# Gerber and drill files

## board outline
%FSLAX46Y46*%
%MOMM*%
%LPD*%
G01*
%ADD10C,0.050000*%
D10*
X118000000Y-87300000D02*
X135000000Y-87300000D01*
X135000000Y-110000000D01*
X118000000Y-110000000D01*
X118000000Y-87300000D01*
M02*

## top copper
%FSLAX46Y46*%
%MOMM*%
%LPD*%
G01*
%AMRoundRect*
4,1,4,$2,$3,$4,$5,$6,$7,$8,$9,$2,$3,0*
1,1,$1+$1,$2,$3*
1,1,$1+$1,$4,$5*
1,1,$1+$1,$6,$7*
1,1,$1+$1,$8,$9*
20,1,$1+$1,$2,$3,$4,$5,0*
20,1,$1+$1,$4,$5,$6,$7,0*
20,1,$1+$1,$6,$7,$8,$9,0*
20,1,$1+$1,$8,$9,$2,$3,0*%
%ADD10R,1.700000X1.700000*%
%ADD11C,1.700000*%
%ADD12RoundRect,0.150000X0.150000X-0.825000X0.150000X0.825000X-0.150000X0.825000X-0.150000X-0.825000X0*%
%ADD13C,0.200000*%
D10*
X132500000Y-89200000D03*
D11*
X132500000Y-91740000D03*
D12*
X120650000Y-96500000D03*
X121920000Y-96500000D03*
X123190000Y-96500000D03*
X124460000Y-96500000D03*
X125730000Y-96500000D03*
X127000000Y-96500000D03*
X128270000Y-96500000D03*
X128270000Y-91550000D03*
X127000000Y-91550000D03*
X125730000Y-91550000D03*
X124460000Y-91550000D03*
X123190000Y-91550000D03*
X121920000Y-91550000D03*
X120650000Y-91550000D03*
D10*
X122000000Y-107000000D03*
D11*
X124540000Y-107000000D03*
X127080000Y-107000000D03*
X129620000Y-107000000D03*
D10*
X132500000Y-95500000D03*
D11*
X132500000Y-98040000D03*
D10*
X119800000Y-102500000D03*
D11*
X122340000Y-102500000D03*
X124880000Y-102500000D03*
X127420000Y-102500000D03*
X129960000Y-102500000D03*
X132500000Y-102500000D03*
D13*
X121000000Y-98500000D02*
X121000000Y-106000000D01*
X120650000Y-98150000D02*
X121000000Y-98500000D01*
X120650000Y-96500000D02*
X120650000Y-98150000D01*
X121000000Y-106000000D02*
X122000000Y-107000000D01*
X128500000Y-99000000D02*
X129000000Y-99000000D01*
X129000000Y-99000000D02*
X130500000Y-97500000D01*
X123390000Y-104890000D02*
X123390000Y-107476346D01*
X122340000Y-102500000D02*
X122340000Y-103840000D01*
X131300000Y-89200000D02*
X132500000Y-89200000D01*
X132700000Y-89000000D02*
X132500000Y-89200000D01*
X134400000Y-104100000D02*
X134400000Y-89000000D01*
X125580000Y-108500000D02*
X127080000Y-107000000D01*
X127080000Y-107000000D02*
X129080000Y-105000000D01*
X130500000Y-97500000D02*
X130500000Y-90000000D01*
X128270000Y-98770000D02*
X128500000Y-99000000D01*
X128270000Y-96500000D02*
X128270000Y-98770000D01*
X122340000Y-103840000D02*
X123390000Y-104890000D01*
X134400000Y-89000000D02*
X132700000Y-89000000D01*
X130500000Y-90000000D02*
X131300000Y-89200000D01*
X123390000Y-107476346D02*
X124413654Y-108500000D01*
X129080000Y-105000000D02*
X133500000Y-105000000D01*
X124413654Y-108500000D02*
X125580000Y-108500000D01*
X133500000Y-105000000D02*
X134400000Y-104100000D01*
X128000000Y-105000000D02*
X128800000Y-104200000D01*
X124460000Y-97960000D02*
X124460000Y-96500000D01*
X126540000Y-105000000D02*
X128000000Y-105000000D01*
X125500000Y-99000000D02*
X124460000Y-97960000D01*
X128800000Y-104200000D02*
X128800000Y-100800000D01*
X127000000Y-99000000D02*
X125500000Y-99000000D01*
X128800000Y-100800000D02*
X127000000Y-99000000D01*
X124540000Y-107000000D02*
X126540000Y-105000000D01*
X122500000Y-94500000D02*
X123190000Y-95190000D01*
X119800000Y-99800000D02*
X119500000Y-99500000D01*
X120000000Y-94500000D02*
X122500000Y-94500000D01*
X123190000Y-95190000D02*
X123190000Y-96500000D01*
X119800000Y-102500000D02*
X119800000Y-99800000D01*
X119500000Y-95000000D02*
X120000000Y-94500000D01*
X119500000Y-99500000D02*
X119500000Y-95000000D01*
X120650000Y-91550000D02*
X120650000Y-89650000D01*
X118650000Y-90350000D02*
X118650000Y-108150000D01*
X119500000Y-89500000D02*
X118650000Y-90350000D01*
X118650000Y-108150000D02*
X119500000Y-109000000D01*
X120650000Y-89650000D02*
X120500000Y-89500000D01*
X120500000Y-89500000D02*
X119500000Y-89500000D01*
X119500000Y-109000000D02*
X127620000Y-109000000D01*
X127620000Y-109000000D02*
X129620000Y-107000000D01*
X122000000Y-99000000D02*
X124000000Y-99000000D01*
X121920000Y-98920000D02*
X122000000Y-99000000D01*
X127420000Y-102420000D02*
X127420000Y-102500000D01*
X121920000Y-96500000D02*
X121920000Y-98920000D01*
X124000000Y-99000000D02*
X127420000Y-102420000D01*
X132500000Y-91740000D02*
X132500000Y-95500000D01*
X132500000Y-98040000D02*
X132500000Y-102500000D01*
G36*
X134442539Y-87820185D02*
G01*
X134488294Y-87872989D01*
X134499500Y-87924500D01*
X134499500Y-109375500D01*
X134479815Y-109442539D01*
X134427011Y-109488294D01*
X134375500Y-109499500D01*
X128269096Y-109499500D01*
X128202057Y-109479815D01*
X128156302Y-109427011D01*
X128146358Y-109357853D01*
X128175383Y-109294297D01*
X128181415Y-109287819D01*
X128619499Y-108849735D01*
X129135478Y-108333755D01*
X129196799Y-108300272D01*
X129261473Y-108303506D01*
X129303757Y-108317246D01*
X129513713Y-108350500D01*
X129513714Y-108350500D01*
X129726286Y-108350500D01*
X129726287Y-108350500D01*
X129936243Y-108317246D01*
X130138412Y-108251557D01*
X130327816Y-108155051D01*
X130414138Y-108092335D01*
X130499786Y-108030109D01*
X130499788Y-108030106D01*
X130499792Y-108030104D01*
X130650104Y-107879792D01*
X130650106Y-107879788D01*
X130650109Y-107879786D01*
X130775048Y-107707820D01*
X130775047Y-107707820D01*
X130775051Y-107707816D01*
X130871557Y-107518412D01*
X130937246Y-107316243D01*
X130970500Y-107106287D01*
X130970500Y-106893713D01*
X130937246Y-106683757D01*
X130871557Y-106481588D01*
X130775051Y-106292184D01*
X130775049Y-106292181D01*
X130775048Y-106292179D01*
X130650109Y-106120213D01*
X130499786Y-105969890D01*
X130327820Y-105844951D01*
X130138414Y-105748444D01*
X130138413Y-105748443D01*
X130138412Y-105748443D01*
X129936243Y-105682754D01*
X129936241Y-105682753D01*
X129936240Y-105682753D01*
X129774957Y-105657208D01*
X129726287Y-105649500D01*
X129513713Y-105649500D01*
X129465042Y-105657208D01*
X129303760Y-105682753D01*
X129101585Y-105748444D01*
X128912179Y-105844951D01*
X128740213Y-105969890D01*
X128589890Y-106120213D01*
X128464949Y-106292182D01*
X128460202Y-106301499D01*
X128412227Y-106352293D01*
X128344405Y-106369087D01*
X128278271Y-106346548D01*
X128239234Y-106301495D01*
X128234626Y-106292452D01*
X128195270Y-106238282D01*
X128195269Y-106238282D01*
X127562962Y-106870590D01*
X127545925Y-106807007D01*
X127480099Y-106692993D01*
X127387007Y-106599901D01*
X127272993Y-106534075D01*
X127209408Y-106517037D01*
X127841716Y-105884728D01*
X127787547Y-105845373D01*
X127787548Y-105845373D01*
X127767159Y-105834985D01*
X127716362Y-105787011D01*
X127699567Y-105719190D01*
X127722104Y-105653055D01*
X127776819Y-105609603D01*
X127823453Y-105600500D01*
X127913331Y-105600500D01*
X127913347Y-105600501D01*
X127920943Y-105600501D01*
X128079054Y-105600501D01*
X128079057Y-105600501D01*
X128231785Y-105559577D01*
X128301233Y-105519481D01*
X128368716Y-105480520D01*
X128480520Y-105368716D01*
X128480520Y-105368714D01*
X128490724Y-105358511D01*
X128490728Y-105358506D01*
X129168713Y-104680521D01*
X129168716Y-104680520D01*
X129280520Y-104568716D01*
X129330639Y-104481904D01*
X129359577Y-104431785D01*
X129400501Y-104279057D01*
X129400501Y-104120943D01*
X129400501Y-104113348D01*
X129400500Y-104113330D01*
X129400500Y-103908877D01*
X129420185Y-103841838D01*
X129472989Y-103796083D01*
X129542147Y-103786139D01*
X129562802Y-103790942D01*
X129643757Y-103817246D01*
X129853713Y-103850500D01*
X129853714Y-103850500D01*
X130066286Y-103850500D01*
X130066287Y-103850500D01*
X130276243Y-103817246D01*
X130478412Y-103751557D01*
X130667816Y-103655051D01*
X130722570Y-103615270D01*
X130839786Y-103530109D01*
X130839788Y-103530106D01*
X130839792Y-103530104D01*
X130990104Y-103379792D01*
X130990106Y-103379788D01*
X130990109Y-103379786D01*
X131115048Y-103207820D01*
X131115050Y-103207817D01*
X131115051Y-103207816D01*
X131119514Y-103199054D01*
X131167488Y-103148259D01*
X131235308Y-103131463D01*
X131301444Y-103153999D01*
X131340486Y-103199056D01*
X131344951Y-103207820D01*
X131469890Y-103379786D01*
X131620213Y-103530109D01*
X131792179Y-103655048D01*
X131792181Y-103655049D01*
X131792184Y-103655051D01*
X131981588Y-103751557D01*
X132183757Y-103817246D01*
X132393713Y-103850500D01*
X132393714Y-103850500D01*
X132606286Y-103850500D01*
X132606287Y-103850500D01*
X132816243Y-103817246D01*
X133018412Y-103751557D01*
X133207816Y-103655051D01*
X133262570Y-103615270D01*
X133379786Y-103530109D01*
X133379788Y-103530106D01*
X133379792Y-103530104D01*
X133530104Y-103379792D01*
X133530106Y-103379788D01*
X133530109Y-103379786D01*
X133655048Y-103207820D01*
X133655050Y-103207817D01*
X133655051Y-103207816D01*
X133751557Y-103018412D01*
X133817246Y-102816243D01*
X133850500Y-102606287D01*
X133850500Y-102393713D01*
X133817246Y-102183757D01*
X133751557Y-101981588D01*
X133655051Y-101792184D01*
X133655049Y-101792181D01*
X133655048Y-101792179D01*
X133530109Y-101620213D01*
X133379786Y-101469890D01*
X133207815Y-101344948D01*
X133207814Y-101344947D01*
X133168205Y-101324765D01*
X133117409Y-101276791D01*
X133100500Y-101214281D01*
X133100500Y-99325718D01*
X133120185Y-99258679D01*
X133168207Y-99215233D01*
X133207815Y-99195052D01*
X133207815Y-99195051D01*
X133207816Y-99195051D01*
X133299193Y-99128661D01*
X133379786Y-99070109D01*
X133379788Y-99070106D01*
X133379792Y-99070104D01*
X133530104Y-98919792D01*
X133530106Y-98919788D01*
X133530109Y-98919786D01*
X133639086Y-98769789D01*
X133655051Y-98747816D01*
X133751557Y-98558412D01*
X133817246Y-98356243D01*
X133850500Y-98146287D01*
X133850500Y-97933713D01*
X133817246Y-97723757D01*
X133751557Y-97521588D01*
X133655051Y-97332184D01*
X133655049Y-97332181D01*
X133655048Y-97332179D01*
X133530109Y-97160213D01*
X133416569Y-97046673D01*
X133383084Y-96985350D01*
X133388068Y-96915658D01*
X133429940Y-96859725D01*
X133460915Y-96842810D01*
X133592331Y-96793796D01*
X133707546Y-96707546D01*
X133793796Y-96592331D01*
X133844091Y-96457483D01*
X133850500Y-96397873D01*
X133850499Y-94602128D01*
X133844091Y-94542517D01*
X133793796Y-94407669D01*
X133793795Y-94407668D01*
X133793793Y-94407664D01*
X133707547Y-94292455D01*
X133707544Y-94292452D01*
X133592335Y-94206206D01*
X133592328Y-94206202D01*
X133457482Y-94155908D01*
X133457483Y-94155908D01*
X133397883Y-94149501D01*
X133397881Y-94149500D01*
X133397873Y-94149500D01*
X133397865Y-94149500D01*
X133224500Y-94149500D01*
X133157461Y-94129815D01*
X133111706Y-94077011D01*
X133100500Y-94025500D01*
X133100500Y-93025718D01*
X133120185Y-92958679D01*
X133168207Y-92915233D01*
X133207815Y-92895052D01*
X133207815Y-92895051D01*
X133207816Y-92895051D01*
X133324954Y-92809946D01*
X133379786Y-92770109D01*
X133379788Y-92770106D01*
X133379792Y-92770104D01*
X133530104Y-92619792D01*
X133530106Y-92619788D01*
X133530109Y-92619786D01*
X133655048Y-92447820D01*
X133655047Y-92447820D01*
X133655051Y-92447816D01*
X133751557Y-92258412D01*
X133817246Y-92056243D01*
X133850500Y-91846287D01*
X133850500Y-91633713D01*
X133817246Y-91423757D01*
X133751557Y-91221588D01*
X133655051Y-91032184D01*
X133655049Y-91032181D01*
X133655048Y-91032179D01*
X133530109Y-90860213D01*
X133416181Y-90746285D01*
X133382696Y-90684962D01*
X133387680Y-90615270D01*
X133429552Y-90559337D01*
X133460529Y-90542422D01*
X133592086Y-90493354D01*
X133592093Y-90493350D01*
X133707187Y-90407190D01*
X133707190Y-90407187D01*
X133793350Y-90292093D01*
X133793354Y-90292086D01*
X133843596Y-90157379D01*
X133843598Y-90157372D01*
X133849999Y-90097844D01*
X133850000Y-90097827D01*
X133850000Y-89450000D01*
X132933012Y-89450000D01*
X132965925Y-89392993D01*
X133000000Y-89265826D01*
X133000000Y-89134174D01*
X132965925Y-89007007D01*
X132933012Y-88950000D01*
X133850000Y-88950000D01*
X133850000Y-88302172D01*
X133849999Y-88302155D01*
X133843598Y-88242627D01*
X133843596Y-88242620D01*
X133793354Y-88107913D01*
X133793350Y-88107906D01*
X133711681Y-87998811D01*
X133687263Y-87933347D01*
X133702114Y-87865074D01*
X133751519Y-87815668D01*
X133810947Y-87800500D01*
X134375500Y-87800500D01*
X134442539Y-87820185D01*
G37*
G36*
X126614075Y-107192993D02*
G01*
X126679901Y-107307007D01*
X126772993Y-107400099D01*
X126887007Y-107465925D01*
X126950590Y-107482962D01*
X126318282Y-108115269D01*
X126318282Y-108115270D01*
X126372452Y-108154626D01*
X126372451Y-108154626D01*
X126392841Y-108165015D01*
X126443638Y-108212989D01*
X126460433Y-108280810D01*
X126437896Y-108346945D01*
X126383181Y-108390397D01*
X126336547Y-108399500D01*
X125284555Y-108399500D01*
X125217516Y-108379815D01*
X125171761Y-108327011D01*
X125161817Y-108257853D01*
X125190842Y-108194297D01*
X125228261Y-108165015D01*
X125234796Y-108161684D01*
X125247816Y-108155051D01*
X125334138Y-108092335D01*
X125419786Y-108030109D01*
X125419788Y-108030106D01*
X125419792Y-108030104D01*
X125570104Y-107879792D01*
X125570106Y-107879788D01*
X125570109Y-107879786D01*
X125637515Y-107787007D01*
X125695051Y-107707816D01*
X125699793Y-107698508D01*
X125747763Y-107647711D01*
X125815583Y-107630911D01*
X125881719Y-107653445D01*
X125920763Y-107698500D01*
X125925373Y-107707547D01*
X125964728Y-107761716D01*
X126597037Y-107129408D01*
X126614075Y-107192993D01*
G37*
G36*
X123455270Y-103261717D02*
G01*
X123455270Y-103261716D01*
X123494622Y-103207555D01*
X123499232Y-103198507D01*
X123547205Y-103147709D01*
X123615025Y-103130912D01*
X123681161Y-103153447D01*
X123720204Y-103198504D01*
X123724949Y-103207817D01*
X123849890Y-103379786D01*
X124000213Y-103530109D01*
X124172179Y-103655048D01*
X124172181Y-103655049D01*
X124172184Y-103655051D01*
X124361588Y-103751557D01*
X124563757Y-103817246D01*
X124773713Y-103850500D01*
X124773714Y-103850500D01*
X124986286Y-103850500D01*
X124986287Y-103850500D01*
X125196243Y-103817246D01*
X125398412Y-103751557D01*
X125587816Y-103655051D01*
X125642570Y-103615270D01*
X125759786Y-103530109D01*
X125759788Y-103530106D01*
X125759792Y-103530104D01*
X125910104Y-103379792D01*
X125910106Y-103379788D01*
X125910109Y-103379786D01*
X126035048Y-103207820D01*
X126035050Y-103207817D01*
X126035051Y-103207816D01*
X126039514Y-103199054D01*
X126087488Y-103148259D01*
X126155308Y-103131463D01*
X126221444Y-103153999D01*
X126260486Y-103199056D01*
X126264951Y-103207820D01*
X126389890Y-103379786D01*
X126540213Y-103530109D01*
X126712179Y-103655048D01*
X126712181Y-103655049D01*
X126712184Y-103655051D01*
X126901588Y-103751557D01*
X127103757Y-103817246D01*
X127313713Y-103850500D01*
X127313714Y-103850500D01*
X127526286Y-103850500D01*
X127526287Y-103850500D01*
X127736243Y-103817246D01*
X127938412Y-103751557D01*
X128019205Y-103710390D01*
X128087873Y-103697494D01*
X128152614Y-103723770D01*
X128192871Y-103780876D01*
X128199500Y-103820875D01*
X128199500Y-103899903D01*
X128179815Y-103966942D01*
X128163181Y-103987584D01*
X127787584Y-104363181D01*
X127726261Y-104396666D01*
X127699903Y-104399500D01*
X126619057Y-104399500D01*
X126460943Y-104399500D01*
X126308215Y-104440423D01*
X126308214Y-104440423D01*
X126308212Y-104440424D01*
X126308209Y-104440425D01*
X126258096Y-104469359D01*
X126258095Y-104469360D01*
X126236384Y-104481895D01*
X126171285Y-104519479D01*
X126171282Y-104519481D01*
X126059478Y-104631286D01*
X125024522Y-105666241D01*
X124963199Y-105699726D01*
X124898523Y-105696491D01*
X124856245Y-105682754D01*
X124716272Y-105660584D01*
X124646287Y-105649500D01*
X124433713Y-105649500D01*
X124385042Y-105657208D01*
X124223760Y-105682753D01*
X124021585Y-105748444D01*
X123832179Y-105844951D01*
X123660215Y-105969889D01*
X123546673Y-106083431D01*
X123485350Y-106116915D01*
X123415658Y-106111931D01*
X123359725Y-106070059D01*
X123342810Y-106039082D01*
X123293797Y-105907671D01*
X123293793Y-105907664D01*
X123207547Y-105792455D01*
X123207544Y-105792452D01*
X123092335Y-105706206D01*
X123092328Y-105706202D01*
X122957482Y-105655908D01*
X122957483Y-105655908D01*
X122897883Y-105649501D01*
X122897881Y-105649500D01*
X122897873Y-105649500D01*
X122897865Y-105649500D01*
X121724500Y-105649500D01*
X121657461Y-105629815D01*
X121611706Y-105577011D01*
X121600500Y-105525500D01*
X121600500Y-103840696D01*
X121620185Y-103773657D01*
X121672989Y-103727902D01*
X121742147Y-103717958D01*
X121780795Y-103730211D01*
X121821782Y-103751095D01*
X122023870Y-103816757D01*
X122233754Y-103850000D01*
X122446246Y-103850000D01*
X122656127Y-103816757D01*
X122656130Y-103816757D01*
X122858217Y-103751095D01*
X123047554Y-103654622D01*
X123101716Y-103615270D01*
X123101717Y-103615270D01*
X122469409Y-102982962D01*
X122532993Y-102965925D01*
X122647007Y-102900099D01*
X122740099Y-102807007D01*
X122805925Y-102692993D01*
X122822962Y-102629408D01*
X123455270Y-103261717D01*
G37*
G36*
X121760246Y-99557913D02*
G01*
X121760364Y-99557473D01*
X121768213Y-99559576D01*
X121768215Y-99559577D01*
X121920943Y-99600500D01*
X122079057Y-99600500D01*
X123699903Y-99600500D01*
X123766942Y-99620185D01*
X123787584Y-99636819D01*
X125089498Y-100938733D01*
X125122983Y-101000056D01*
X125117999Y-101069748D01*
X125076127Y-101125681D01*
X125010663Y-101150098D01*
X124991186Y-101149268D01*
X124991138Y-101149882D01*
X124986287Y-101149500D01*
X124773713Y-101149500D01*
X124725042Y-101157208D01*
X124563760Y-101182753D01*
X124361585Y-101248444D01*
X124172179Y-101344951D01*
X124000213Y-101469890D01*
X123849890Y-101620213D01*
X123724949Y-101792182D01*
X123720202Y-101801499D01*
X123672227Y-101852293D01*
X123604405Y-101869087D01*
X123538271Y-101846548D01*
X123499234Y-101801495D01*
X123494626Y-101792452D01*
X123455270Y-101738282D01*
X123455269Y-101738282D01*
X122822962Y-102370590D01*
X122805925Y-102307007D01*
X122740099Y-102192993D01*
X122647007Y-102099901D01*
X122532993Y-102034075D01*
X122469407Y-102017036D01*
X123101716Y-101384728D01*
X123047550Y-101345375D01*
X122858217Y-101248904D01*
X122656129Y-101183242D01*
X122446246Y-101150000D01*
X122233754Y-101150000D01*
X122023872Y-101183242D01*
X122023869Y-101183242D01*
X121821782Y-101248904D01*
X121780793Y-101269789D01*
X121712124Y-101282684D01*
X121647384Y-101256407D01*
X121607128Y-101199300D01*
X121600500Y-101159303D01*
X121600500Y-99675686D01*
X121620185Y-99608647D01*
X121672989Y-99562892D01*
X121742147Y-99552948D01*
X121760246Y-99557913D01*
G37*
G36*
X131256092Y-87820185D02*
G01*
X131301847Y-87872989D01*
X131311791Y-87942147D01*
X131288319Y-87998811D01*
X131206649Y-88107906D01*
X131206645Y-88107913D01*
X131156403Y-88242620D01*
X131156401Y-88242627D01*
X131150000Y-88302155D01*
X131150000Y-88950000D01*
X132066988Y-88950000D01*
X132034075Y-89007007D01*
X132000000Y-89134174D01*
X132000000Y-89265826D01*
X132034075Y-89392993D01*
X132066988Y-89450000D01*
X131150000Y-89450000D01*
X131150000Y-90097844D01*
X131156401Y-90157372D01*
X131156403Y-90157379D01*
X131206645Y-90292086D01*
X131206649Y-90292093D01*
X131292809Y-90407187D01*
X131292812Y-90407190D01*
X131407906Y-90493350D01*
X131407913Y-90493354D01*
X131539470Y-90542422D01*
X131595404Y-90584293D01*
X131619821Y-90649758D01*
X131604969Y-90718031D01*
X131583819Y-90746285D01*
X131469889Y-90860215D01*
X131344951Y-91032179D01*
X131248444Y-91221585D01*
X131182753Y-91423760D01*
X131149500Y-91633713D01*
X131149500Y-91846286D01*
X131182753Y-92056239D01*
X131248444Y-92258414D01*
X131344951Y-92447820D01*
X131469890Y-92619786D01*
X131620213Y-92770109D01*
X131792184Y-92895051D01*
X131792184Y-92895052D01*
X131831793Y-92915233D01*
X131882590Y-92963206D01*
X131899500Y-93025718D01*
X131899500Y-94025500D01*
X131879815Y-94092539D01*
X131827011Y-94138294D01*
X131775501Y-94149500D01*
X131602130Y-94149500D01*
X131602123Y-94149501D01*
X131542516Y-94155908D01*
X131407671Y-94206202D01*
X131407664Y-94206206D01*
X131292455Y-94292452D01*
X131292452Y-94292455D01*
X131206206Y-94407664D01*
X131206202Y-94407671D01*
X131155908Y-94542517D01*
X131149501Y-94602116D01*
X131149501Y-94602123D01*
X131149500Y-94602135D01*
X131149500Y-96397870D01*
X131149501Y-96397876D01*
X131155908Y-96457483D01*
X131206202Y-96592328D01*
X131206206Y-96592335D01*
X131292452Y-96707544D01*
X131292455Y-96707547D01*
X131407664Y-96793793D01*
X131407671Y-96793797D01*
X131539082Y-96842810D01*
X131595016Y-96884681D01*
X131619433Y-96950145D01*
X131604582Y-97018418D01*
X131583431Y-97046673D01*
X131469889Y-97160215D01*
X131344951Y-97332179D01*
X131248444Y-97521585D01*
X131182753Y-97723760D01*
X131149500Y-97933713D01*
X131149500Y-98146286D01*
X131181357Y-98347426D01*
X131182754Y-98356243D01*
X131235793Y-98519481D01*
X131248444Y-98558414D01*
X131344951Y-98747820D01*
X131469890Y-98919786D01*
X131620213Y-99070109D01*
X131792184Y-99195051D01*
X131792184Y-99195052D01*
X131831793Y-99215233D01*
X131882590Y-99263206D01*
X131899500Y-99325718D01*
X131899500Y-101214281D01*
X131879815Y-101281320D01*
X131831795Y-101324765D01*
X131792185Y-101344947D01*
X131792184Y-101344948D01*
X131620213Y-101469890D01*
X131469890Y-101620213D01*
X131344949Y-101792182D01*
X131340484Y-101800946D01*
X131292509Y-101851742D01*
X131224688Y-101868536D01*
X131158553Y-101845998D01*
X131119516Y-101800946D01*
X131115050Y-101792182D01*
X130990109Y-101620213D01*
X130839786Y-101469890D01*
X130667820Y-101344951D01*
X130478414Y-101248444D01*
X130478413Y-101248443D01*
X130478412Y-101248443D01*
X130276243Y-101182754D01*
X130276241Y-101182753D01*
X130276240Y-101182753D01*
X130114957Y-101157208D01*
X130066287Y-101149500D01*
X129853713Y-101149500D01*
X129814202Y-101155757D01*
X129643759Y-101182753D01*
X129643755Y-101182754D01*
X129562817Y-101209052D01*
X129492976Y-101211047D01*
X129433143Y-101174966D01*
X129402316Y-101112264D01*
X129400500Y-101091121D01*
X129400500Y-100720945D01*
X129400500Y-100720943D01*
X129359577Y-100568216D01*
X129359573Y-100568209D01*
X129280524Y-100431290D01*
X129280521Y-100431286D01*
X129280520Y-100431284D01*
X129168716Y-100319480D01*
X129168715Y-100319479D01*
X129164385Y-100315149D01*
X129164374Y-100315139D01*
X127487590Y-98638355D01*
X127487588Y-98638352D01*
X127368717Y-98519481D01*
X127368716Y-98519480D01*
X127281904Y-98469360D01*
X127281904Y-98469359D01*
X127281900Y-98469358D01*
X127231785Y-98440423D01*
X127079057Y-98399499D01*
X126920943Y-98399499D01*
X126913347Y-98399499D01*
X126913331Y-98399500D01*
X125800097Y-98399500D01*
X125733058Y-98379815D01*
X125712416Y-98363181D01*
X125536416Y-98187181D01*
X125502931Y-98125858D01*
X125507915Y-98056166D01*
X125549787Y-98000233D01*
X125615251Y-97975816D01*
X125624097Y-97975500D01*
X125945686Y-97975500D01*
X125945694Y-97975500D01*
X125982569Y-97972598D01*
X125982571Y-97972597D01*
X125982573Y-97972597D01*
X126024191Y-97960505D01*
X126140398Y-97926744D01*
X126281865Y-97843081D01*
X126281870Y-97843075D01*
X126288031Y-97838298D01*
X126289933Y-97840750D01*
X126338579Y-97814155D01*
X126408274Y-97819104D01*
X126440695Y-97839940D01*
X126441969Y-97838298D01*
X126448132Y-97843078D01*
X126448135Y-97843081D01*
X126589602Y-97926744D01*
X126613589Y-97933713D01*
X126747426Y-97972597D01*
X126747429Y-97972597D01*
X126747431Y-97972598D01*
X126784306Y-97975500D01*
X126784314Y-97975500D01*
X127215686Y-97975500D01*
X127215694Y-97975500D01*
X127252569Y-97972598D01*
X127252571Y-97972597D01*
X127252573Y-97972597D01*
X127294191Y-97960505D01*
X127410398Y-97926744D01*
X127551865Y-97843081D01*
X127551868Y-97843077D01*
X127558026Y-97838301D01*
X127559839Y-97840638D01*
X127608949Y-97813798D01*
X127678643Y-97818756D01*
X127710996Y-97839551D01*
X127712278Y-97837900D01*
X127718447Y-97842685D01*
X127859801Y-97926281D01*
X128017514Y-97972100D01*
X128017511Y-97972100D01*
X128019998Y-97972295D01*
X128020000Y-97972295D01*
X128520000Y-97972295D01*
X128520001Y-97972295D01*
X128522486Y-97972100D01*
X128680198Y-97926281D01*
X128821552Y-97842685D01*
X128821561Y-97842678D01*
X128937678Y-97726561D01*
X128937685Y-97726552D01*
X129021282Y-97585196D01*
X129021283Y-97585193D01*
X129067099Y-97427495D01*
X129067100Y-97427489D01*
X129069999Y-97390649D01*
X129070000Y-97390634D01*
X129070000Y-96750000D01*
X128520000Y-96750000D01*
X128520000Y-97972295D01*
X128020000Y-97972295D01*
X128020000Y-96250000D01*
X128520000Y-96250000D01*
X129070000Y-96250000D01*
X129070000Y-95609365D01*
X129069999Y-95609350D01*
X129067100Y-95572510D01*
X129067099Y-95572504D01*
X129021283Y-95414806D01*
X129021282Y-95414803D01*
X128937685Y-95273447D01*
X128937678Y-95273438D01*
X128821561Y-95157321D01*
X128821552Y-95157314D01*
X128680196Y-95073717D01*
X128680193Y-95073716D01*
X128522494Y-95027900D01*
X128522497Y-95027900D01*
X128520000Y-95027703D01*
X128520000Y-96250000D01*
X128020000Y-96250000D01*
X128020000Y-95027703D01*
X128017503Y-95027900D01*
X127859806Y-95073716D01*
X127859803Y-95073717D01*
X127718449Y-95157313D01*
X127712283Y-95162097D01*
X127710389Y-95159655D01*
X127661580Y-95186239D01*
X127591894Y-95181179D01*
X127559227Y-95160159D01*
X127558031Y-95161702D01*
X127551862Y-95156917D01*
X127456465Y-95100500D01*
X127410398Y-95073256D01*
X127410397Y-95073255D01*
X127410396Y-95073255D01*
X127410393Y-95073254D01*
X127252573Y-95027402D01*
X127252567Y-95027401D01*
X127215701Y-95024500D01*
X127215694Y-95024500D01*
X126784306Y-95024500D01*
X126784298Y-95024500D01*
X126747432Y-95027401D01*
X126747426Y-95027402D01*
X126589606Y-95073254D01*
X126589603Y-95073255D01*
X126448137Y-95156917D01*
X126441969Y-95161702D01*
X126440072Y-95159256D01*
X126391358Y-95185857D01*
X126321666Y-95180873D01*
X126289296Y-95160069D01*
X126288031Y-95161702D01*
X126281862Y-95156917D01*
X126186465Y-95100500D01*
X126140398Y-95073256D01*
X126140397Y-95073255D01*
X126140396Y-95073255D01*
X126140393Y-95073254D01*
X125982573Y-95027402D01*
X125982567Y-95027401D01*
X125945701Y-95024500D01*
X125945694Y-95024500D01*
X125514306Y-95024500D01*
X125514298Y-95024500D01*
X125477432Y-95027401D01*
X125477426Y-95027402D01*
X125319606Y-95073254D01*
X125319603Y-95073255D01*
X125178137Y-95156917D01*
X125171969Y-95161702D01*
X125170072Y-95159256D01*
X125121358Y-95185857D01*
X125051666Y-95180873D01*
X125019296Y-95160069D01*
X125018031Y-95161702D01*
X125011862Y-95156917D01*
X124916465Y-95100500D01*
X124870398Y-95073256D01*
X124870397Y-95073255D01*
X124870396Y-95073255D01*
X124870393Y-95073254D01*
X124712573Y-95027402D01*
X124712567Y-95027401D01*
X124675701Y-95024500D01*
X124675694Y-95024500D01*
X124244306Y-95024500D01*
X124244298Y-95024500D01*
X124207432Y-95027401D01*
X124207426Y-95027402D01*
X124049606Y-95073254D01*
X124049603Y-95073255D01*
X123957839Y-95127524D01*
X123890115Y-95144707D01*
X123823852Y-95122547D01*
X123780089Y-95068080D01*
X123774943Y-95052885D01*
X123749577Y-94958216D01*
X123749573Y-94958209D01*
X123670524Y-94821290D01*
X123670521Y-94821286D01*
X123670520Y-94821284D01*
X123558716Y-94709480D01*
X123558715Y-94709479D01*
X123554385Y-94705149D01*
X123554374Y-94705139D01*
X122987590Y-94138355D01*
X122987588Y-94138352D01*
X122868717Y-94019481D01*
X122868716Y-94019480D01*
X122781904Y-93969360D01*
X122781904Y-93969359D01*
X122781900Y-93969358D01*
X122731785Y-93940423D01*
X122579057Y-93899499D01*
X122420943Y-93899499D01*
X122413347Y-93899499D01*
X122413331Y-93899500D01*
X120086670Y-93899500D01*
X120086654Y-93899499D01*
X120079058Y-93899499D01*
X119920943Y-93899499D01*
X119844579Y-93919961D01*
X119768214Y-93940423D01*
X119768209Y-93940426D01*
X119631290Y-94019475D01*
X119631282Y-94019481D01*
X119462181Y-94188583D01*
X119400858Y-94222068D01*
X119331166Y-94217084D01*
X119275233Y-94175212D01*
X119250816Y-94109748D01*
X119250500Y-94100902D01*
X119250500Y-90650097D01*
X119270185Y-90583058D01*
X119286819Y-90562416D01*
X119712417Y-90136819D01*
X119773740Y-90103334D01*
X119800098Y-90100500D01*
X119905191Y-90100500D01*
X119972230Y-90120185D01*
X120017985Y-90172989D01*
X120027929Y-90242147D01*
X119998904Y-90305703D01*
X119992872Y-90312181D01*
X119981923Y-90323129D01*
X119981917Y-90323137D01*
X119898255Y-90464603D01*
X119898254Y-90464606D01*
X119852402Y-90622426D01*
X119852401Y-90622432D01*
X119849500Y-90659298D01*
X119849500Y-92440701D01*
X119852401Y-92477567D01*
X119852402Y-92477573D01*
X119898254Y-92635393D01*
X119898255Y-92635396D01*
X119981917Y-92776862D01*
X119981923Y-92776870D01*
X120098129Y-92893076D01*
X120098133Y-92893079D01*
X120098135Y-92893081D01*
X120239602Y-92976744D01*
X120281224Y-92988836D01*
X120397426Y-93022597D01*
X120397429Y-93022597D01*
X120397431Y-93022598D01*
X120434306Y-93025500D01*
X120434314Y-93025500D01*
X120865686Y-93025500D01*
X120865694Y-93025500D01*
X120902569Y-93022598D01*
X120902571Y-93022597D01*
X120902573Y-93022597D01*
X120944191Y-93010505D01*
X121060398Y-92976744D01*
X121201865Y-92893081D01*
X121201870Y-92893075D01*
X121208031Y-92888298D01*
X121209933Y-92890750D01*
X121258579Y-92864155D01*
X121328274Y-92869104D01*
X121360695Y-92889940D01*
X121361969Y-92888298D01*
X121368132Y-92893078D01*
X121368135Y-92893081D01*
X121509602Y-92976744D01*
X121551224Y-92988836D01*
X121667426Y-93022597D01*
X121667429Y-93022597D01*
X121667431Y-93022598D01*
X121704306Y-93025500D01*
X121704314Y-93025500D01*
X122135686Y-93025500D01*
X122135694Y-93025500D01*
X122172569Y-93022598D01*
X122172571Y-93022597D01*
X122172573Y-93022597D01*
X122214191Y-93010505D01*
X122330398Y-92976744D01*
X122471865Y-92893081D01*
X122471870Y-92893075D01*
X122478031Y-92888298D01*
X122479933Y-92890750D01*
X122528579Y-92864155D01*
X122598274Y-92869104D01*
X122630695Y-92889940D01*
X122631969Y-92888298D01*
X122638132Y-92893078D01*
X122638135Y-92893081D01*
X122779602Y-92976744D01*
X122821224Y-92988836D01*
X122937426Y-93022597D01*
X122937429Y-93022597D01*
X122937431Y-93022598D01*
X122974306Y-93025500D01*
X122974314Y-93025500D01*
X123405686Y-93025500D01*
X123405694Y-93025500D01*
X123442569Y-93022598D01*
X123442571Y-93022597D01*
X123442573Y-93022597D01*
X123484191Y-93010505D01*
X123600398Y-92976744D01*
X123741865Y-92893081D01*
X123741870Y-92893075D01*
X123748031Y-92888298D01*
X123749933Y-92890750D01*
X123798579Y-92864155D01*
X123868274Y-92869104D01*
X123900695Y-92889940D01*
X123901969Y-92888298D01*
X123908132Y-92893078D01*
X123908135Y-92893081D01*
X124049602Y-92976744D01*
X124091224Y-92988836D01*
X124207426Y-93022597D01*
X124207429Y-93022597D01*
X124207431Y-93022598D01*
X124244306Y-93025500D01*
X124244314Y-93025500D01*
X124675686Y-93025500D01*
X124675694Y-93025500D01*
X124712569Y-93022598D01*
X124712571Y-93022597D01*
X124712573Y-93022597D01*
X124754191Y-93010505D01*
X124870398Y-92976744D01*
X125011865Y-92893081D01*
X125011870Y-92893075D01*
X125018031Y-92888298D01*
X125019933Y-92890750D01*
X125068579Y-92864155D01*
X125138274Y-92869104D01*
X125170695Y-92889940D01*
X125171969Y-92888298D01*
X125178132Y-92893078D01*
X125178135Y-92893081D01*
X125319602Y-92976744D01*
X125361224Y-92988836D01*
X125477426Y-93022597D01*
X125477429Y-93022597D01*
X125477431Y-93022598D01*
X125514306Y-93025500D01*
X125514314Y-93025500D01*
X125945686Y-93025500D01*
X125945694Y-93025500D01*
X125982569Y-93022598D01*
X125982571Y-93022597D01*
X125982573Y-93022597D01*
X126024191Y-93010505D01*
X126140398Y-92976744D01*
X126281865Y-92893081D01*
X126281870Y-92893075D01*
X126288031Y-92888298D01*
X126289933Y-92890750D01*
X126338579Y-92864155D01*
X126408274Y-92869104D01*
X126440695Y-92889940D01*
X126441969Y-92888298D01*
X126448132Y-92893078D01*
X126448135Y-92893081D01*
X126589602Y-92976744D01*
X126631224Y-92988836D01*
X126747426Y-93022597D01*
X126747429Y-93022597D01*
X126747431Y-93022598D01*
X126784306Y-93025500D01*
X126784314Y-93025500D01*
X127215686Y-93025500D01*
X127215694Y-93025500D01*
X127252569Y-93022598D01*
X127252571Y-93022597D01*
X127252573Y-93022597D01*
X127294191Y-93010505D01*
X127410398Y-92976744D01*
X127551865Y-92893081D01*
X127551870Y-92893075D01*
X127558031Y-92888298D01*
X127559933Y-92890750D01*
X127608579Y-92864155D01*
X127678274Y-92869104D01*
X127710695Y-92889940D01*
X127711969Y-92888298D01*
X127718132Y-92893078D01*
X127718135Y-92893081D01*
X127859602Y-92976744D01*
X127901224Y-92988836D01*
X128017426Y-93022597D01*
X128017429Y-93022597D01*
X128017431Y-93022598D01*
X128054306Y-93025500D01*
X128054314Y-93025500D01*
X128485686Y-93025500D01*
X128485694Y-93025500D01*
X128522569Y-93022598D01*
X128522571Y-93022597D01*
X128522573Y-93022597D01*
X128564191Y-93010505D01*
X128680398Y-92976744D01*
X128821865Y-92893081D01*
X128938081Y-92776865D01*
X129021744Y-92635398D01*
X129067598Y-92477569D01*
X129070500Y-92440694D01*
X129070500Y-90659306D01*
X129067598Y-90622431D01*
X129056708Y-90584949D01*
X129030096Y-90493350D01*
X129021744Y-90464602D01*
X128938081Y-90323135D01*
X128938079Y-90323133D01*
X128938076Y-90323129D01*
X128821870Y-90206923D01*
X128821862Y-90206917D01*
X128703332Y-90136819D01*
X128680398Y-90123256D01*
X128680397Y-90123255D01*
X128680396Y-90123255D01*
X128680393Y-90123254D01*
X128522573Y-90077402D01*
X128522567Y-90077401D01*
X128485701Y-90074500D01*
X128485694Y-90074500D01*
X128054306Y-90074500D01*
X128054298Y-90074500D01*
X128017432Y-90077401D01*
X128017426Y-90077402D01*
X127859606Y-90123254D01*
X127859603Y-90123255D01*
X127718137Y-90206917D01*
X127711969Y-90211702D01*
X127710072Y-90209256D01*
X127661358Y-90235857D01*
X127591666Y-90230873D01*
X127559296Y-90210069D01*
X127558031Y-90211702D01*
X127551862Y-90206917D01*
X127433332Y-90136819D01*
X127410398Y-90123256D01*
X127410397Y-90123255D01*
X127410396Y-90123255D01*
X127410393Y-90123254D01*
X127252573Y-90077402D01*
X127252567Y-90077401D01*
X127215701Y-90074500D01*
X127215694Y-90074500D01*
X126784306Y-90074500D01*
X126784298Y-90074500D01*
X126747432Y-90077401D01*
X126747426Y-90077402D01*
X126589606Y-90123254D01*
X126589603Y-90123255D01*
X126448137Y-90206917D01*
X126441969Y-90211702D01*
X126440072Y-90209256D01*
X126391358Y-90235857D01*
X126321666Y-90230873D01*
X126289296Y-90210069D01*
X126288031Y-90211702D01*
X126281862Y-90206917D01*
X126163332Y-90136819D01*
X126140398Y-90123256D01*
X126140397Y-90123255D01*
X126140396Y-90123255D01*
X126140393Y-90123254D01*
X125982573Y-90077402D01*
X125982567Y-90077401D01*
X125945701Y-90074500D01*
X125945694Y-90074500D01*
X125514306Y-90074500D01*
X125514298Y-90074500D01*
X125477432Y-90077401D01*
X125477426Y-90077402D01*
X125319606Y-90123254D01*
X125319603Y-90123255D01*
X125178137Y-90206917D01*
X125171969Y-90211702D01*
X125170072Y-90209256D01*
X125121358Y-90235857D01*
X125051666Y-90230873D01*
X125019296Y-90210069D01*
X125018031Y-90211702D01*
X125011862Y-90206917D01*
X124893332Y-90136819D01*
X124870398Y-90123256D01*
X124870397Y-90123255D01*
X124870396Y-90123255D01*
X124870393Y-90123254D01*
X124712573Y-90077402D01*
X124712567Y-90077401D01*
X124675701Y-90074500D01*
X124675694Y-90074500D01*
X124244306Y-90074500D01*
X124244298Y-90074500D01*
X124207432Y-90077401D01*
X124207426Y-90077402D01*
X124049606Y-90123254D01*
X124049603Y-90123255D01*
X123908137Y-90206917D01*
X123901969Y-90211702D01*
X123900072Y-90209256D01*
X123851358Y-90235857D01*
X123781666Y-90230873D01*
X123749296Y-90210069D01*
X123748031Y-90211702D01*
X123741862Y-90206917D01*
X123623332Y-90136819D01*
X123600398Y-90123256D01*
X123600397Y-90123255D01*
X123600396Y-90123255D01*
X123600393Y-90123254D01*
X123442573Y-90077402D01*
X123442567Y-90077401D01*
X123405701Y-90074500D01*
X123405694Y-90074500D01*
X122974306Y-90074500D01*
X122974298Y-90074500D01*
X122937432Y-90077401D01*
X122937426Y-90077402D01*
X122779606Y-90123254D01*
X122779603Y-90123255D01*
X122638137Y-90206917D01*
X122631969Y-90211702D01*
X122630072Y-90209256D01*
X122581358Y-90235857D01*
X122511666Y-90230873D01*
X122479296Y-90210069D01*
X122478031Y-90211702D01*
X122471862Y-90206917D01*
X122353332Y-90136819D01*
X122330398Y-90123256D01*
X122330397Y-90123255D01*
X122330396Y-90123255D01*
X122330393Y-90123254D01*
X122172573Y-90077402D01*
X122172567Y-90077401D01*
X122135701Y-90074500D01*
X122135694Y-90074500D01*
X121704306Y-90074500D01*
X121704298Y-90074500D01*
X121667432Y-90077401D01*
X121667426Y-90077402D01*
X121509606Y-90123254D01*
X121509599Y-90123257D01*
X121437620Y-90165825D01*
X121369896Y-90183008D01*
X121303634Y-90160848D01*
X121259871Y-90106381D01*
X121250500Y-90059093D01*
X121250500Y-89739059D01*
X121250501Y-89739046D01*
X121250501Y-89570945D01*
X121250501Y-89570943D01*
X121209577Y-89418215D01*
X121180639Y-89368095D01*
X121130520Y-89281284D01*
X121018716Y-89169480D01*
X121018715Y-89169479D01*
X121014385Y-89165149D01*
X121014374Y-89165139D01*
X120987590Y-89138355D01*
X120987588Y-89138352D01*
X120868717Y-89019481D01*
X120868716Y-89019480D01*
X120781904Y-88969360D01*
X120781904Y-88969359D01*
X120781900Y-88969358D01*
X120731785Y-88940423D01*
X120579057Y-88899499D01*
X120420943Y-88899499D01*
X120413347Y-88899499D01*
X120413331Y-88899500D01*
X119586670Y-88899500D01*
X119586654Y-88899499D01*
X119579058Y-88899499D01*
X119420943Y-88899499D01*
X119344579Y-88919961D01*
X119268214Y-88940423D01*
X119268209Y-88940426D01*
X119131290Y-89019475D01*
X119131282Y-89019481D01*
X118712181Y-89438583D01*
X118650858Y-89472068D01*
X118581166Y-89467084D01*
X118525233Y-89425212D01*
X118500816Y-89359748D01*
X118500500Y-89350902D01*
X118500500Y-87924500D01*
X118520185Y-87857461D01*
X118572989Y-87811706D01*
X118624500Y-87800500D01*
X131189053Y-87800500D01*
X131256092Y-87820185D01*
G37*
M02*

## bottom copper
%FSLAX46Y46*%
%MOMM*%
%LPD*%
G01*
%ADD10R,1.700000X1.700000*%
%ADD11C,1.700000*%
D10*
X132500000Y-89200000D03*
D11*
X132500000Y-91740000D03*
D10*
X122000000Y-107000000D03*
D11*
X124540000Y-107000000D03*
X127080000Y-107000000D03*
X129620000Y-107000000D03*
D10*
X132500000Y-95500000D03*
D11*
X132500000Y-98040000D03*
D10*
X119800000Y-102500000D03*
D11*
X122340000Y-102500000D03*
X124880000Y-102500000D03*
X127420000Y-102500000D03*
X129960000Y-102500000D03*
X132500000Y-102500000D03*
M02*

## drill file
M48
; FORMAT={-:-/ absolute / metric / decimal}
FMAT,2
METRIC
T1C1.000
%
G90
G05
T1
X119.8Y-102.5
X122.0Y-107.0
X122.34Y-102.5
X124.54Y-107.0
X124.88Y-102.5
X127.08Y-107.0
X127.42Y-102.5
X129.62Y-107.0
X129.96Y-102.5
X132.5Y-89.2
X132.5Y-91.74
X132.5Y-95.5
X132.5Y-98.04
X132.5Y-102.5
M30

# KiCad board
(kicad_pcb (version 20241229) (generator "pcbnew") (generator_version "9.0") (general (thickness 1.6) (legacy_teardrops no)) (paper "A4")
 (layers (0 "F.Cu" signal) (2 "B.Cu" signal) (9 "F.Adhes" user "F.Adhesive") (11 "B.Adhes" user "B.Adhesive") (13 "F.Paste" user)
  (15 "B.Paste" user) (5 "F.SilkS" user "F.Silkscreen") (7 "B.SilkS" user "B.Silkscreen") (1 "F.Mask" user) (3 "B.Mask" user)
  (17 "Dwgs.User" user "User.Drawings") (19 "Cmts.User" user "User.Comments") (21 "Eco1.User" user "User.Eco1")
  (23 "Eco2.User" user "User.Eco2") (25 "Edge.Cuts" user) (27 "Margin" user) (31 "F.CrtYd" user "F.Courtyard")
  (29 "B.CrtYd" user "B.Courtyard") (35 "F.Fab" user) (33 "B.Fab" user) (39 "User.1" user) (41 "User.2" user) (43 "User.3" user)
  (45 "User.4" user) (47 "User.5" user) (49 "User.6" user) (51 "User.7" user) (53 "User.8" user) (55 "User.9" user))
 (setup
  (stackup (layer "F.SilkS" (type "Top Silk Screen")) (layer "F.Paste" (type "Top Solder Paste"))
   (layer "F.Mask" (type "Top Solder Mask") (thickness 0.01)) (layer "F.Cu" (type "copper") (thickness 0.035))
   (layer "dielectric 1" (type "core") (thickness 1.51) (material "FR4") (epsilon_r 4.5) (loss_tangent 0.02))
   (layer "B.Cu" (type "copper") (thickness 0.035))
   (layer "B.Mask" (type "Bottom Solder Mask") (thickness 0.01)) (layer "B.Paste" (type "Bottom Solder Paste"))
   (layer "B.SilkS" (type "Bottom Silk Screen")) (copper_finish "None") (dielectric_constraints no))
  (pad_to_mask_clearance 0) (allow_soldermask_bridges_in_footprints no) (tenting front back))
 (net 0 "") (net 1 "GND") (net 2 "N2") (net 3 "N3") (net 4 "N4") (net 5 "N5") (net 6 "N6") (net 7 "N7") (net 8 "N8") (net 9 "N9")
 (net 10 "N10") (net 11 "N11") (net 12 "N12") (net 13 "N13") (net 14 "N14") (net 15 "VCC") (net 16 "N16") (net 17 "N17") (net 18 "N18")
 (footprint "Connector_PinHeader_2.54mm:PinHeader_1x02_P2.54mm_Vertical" (layer "F.Cu") (at 132.5 89.2)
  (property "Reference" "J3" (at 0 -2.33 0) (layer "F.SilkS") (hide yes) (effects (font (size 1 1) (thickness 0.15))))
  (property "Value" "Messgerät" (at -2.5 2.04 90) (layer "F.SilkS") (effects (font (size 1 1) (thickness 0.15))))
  (pad "1" thru_hole rect (at 0 0) (size 1.7 1.7) (drill 1) (layers "*.Cu" "*.Mask") (remove_unused_layers no) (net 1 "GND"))
  (pad "2" thru_hole circle (at 0 2.54) (size 1.7 1.7) (drill 1) (layers "*.Cu" "*.Mask") (remove_unused_layers no) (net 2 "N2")))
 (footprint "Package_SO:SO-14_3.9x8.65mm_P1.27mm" (layer "F.Cu") (at 124.46 94.025 90)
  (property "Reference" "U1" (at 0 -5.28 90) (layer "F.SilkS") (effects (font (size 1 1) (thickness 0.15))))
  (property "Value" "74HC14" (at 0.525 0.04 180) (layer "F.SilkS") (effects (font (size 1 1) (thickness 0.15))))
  (pad "1" smd roundrect (at -2.475 -3.81 90) (size 1.95 0.6) (layers "F.Cu" "F.Mask" "F.Paste") (roundrect_rratio 0.25) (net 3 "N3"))
  (pad "2" smd roundrect (at -2.475 -2.54 90) (size 1.95 0.6) (layers "F.Cu" "F.Mask" "F.Paste") (roundrect_rratio 0.25) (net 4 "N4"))
  (pad "3" smd roundrect (at -2.475 -1.27 90) (size 1.95 0.6) (layers "F.Cu" "F.Mask" "F.Paste") (roundrect_rratio 0.25) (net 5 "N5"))
  (pad "4" smd roundrect (at -2.475 0 90) (size 1.95 0.6) (layers "F.Cu" "F.Mask" "F.Paste") (roundrect_rratio 0.25) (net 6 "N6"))
  (pad "5" smd roundrect (at -2.475 1.27 90) (size 1.95 0.6) (layers "F.Cu" "F.Mask" "F.Paste") (roundrect_rratio 0.25) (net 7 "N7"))
  (pad "6" smd roundrect (at -2.475 2.54 90) (size 1.95 0.6) (layers "F.Cu" "F.Mask" "F.Paste") (roundrect_rratio 0.25) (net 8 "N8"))
  (pad "7" smd roundrect (at -2.475 3.81 90) (size 1.95 0.6) (layers "F.Cu" "F.Mask" "F.Paste") (roundrect_rratio 0.25) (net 1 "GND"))
  (pad "8" smd roundrect (at 2.475 3.81 90) (size 1.95 0.6) (layers "F.Cu" "F.Mask" "F.Paste") (roundrect_rratio 0.25) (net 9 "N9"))
  (pad "9" smd roundrect (at 2.475 2.54 90) (size 1.95 0.6) (layers "F.Cu" "F.Mask" "F.Paste") (roundrect_rratio 0.25) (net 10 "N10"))
  (pad "10" smd roundrect (at 2.475 1.27 90) (size 1.95 0.6) (layers "F.Cu" "F.Mask" "F.Paste") (roundrect_rratio 0.25) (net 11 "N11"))
  (pad "11" smd roundrect (at 2.475 0 90) (size 1.95 0.6) (layers "F.Cu" "F.Mask" "F.Paste") (roundrect_rratio 0.25) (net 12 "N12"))
  (pad "12" smd roundrect (at 2.475 -1.27 90) (size 1.95 0.6) (layers "F.Cu" "F.Mask" "F.Paste") (roundrect_rratio 0.25) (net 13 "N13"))
  (pad "13" smd roundrect (at 2.475 -2.54 90) (size 1.95 0.6) (layers "F.Cu" "F.Mask" "F.Paste") (roundrect_rratio 0.25) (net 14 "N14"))
  (pad "14" smd roundrect (at 2.475 -3.81 90) (size 1.95 0.6) (layers "F.Cu" "F.Mask" "F.Paste") (roundrect_rratio 0.25) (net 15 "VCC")))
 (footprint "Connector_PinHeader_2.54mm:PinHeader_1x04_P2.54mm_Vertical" (layer "F.Cu") (at 122 107 90)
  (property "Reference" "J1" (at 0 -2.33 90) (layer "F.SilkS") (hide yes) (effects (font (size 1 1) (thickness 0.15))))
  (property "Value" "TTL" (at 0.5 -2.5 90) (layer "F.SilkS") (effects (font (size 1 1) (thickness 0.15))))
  (pad "1" thru_hole rect (at 0 0 90) (size 1.7 1.7) (drill 1) (layers "*.Cu" "*.Mask") (remove_unused_layers no) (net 3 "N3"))
  (pad "2" thru_hole circle (at 0 2.54 90) (size 1.7 1.7) (drill 1) (layers "*.Cu" "*.Mask") (remove_unused_layers no) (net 6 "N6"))
  (pad "3" thru_hole circle (at 0 5.08 90) (size 1.7 1.7) (drill 1) (layers "*.Cu" "*.Mask") (remove_unused_layers no) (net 1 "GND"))
  (pad "4" thru_hole circle (at 0 7.62 90) (size 1.7 1.7) (drill 1) (layers "*.Cu" "*.Mask") (remove_unused_layers no) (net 15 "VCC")))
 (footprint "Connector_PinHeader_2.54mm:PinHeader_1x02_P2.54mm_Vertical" (layer "F.Cu") (at 132.5 95.5)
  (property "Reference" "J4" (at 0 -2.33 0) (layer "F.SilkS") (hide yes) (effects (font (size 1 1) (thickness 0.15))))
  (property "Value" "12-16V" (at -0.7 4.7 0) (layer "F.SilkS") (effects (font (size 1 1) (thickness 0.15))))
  (pad "1" thru_hole rect (at 0 0) (size 1.7 1.7) (drill 1) (layers "*.Cu" "*.Mask") (remove_unused_layers no) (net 2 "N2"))
  (pad "2" thru_hole circle (at 0 2.54) (size 1.7 1.7) (drill 1) (layers "*.Cu" "*.Mask") (remove_unused_layers no) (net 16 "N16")))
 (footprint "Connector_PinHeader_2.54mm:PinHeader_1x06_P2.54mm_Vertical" (layer "F.Cu") (at 119.8 102.5 90)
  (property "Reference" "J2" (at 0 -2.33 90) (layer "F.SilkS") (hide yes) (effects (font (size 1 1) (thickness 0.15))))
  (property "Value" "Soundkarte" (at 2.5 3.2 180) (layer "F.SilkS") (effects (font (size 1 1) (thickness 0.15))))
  (pad "1" thru_hole rect (at 0 0 90) (size 1.7 1.7) (drill 1) (layers "*.Cu" "*.Mask") (remove_unused_layers no) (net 5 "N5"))
  (pad "2" thru_hole circle (at 0 2.54 90) (size 1.7 1.7) (drill 1) (layers "*.Cu" "*.Mask") (remove_unused_layers no) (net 1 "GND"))
  (pad "3" thru_hole circle (at 0 5.08 90) (size 1.7 1.7) (drill 1) (layers "*.Cu" "*.Mask") (remove_unused_layers no) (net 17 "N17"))
  (pad "4" thru_hole circle (at 0 7.62 90) (size 1.7 1.7) (drill 1) (layers "*.Cu" "*.Mask") (remove_unused_layers no) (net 4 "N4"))
  (pad "5" thru_hole circle (at 0 10.16 90) (size 1.7 1.7) (drill 1) (layers "*.Cu" "*.Mask") (remove_unused_layers no) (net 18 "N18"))
  (pad "6" thru_hole circle (at 0 12.7 90) (size 1.7 1.7) (drill 1) (layers "*.Cu" "*.Mask") (remove_unused_layers no) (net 16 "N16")))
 (gr_rect (start 118 87.3) (end 135 110) (stroke (width 0.05) (type default)) (fill no) (layer "Edge.Cuts"))
 (segment (start 121 98.5) (end 121 106) (width 0.2) (layer "F.Cu") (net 3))
 (segment (start 120.65 98.15) (end 121 98.5) (width 0.2) (layer "F.Cu") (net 3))
 (segment (start 120.65 96.5) (end 120.65 98.15) (width 0.2) (layer "F.Cu") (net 3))
 (segment (start 121 106) (end 122 107) (width 0.2) (layer "F.Cu") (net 3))
 (segment (start 128.5 99) (end 129 99) (width 0.2) (layer "F.Cu") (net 1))
 (segment (start 129 99) (end 130.5 97.5) (width 0.2) (layer "F.Cu") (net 1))
 (segment (start 123.39 104.89) (end 123.39 107.476346) (width 0.2) (layer "F.Cu") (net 1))
 (segment (start 122.34 102.5) (end 122.34 103.84) (width 0.2) (layer "F.Cu") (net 1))
 (segment (start 131.3 89.2) (end 132.5 89.2) (width 0.2) (layer "F.Cu") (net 1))
 (segment (start 132.7 89) (end 132.5 89.2) (width 0.2) (layer "F.Cu") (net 1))
 (segment (start 134.4 104.1) (end 134.4 89) (width 0.2) (layer "F.Cu") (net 1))
 (segment (start 125.58 108.5) (end 127.08 107) (width 0.2) (layer "F.Cu") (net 1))
 (segment (start 127.08 107) (end 129.08 105) (width 0.2) (layer "F.Cu") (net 1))
 (segment (start 130.5 97.5) (end 130.5 90) (width 0.2) (layer "F.Cu") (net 1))
 (segment (start 128.27 98.77) (end 128.5 99) (width 0.2) (layer "F.Cu") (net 1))
 (segment (start 128.27 96.5) (end 128.27 98.77) (width 0.2) (layer "F.Cu") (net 1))
 (segment (start 122.34 103.84) (end 123.39 104.89) (width 0.2) (layer "F.Cu") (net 1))
 (segment (start 134.4 89) (end 132.7 89) (width 0.2) (layer "F.Cu") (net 1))
 (segment (start 130.5 90) (end 131.3 89.2) (width 0.2) (layer "F.Cu") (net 1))
 (segment (start 123.39 107.476346) (end 124.413654 108.5) (width 0.2) (layer "F.Cu") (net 1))
 (segment (start 129.08 105) (end 133.5 105) (width 0.2) (layer "F.Cu") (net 1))
 (segment (start 124.413654 108.5) (end 125.58 108.5) (width 0.2) (layer "F.Cu") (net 1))
 (segment (start 133.5 105) (end 134.4 104.1) (width 0.2) (layer "F.Cu") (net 1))
 (segment (start 128 105) (end 128.8 104.2) (width 0.2) (layer "F.Cu") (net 6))
 (segment (start 124.46 97.96) (end 124.46 96.5) (width 0.2) (layer "F.Cu") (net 6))
 (segment (start 126.54 105) (end 128 105) (width 0.2) (layer "F.Cu") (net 6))
 (segment (start 125.5 99) (end 124.46 97.96) (width 0.2) (layer "F.Cu") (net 6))
 (segment (start 128.8 104.2) (end 128.8 100.8) (width 0.2) (layer "F.Cu") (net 6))
 (segment (start 127 99) (end 125.5 99) (width 0.2) (layer "F.Cu") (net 6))
 (segment (start 128.8 100.8) (end 127 99) (width 0.2) (layer "F.Cu") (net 6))
 (segment (start 124.54 107) (end 126.54 105) (width 0.2) (layer "F.Cu") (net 6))
 (segment (start 122.5 94.5) (end 123.19 95.19) (width 0.2) (layer "F.Cu") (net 5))
 (segment (start 119.8 99.8) (end 119.5 99.5) (width 0.2) (layer "F.Cu") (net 5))
 (segment (start 120 94.5) (end 122.5 94.5) (width 0.2) (layer "F.Cu") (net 5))
 (segment (start 123.19 95.19) (end 123.19 96.5) (width 0.2) (layer "F.Cu") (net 5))
 (segment (start 119.8 102.5) (end 119.8 99.8) (width 0.2) (layer "F.Cu") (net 5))
 (segment (start 119.5 95) (end 120 94.5) (width 0.2) (layer "F.Cu") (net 5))
 (segment (start 119.5 99.5) (end 119.5 95) (width 0.2) (layer "F.Cu") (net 5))
 (segment (start 120.65 91.55) (end 120.65 89.65) (width 0.2) (layer "F.Cu") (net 15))
 (segment (start 118.65 90.35) (end 118.65 108.15) (width 0.2) (layer "F.Cu") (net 15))
 (segment (start 119.5 89.5) (end 118.65 90.35) (width 0.2) (layer "F.Cu") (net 15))
 (segment (start 118.65 108.15) (end 119.5 109) (width 0.2) (layer "F.Cu") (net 15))
 (segment (start 120.65 89.65) (end 120.5 89.5) (width 0.2) (layer "F.Cu") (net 15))
 (segment (start 120.5 89.5) (end 119.5 89.5) (width 0.2) (layer "F.Cu") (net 15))
 (segment (start 119.5 109) (end 127.62 109) (width 0.2) (layer "F.Cu") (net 15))
 (segment (start 127.62 109) (end 129.62 107) (width 0.2) (layer "F.Cu") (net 15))
 (segment (start 122 99) (end 124 99) (width 0.2) (layer "F.Cu") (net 4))
 (segment (start 121.92 98.92) (end 122 99) (width 0.2) (layer "F.Cu") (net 4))
 (segment (start 127.42 102.42) (end 127.42 102.5) (width 0.2) (layer "F.Cu") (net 4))
 (segment (start 121.92 96.5) (end 121.92 98.92) (width 0.2) (layer "F.Cu") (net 4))
 (segment (start 124 99) (end 127.42 102.42) (width 0.2) (layer "F.Cu") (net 4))
 (segment (start 132.5 91.74) (end 132.5 95.5) (width 0.2) (layer "F.Cu") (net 2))
 (segment (start 132.5 98.04) (end 132.5 102.5) (width 0.2) (layer "F.Cu") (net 16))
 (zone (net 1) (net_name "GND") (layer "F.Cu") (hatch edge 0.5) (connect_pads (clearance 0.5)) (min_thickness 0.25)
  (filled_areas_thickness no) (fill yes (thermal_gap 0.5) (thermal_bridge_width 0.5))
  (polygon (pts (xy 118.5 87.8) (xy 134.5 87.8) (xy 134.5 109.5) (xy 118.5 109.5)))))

